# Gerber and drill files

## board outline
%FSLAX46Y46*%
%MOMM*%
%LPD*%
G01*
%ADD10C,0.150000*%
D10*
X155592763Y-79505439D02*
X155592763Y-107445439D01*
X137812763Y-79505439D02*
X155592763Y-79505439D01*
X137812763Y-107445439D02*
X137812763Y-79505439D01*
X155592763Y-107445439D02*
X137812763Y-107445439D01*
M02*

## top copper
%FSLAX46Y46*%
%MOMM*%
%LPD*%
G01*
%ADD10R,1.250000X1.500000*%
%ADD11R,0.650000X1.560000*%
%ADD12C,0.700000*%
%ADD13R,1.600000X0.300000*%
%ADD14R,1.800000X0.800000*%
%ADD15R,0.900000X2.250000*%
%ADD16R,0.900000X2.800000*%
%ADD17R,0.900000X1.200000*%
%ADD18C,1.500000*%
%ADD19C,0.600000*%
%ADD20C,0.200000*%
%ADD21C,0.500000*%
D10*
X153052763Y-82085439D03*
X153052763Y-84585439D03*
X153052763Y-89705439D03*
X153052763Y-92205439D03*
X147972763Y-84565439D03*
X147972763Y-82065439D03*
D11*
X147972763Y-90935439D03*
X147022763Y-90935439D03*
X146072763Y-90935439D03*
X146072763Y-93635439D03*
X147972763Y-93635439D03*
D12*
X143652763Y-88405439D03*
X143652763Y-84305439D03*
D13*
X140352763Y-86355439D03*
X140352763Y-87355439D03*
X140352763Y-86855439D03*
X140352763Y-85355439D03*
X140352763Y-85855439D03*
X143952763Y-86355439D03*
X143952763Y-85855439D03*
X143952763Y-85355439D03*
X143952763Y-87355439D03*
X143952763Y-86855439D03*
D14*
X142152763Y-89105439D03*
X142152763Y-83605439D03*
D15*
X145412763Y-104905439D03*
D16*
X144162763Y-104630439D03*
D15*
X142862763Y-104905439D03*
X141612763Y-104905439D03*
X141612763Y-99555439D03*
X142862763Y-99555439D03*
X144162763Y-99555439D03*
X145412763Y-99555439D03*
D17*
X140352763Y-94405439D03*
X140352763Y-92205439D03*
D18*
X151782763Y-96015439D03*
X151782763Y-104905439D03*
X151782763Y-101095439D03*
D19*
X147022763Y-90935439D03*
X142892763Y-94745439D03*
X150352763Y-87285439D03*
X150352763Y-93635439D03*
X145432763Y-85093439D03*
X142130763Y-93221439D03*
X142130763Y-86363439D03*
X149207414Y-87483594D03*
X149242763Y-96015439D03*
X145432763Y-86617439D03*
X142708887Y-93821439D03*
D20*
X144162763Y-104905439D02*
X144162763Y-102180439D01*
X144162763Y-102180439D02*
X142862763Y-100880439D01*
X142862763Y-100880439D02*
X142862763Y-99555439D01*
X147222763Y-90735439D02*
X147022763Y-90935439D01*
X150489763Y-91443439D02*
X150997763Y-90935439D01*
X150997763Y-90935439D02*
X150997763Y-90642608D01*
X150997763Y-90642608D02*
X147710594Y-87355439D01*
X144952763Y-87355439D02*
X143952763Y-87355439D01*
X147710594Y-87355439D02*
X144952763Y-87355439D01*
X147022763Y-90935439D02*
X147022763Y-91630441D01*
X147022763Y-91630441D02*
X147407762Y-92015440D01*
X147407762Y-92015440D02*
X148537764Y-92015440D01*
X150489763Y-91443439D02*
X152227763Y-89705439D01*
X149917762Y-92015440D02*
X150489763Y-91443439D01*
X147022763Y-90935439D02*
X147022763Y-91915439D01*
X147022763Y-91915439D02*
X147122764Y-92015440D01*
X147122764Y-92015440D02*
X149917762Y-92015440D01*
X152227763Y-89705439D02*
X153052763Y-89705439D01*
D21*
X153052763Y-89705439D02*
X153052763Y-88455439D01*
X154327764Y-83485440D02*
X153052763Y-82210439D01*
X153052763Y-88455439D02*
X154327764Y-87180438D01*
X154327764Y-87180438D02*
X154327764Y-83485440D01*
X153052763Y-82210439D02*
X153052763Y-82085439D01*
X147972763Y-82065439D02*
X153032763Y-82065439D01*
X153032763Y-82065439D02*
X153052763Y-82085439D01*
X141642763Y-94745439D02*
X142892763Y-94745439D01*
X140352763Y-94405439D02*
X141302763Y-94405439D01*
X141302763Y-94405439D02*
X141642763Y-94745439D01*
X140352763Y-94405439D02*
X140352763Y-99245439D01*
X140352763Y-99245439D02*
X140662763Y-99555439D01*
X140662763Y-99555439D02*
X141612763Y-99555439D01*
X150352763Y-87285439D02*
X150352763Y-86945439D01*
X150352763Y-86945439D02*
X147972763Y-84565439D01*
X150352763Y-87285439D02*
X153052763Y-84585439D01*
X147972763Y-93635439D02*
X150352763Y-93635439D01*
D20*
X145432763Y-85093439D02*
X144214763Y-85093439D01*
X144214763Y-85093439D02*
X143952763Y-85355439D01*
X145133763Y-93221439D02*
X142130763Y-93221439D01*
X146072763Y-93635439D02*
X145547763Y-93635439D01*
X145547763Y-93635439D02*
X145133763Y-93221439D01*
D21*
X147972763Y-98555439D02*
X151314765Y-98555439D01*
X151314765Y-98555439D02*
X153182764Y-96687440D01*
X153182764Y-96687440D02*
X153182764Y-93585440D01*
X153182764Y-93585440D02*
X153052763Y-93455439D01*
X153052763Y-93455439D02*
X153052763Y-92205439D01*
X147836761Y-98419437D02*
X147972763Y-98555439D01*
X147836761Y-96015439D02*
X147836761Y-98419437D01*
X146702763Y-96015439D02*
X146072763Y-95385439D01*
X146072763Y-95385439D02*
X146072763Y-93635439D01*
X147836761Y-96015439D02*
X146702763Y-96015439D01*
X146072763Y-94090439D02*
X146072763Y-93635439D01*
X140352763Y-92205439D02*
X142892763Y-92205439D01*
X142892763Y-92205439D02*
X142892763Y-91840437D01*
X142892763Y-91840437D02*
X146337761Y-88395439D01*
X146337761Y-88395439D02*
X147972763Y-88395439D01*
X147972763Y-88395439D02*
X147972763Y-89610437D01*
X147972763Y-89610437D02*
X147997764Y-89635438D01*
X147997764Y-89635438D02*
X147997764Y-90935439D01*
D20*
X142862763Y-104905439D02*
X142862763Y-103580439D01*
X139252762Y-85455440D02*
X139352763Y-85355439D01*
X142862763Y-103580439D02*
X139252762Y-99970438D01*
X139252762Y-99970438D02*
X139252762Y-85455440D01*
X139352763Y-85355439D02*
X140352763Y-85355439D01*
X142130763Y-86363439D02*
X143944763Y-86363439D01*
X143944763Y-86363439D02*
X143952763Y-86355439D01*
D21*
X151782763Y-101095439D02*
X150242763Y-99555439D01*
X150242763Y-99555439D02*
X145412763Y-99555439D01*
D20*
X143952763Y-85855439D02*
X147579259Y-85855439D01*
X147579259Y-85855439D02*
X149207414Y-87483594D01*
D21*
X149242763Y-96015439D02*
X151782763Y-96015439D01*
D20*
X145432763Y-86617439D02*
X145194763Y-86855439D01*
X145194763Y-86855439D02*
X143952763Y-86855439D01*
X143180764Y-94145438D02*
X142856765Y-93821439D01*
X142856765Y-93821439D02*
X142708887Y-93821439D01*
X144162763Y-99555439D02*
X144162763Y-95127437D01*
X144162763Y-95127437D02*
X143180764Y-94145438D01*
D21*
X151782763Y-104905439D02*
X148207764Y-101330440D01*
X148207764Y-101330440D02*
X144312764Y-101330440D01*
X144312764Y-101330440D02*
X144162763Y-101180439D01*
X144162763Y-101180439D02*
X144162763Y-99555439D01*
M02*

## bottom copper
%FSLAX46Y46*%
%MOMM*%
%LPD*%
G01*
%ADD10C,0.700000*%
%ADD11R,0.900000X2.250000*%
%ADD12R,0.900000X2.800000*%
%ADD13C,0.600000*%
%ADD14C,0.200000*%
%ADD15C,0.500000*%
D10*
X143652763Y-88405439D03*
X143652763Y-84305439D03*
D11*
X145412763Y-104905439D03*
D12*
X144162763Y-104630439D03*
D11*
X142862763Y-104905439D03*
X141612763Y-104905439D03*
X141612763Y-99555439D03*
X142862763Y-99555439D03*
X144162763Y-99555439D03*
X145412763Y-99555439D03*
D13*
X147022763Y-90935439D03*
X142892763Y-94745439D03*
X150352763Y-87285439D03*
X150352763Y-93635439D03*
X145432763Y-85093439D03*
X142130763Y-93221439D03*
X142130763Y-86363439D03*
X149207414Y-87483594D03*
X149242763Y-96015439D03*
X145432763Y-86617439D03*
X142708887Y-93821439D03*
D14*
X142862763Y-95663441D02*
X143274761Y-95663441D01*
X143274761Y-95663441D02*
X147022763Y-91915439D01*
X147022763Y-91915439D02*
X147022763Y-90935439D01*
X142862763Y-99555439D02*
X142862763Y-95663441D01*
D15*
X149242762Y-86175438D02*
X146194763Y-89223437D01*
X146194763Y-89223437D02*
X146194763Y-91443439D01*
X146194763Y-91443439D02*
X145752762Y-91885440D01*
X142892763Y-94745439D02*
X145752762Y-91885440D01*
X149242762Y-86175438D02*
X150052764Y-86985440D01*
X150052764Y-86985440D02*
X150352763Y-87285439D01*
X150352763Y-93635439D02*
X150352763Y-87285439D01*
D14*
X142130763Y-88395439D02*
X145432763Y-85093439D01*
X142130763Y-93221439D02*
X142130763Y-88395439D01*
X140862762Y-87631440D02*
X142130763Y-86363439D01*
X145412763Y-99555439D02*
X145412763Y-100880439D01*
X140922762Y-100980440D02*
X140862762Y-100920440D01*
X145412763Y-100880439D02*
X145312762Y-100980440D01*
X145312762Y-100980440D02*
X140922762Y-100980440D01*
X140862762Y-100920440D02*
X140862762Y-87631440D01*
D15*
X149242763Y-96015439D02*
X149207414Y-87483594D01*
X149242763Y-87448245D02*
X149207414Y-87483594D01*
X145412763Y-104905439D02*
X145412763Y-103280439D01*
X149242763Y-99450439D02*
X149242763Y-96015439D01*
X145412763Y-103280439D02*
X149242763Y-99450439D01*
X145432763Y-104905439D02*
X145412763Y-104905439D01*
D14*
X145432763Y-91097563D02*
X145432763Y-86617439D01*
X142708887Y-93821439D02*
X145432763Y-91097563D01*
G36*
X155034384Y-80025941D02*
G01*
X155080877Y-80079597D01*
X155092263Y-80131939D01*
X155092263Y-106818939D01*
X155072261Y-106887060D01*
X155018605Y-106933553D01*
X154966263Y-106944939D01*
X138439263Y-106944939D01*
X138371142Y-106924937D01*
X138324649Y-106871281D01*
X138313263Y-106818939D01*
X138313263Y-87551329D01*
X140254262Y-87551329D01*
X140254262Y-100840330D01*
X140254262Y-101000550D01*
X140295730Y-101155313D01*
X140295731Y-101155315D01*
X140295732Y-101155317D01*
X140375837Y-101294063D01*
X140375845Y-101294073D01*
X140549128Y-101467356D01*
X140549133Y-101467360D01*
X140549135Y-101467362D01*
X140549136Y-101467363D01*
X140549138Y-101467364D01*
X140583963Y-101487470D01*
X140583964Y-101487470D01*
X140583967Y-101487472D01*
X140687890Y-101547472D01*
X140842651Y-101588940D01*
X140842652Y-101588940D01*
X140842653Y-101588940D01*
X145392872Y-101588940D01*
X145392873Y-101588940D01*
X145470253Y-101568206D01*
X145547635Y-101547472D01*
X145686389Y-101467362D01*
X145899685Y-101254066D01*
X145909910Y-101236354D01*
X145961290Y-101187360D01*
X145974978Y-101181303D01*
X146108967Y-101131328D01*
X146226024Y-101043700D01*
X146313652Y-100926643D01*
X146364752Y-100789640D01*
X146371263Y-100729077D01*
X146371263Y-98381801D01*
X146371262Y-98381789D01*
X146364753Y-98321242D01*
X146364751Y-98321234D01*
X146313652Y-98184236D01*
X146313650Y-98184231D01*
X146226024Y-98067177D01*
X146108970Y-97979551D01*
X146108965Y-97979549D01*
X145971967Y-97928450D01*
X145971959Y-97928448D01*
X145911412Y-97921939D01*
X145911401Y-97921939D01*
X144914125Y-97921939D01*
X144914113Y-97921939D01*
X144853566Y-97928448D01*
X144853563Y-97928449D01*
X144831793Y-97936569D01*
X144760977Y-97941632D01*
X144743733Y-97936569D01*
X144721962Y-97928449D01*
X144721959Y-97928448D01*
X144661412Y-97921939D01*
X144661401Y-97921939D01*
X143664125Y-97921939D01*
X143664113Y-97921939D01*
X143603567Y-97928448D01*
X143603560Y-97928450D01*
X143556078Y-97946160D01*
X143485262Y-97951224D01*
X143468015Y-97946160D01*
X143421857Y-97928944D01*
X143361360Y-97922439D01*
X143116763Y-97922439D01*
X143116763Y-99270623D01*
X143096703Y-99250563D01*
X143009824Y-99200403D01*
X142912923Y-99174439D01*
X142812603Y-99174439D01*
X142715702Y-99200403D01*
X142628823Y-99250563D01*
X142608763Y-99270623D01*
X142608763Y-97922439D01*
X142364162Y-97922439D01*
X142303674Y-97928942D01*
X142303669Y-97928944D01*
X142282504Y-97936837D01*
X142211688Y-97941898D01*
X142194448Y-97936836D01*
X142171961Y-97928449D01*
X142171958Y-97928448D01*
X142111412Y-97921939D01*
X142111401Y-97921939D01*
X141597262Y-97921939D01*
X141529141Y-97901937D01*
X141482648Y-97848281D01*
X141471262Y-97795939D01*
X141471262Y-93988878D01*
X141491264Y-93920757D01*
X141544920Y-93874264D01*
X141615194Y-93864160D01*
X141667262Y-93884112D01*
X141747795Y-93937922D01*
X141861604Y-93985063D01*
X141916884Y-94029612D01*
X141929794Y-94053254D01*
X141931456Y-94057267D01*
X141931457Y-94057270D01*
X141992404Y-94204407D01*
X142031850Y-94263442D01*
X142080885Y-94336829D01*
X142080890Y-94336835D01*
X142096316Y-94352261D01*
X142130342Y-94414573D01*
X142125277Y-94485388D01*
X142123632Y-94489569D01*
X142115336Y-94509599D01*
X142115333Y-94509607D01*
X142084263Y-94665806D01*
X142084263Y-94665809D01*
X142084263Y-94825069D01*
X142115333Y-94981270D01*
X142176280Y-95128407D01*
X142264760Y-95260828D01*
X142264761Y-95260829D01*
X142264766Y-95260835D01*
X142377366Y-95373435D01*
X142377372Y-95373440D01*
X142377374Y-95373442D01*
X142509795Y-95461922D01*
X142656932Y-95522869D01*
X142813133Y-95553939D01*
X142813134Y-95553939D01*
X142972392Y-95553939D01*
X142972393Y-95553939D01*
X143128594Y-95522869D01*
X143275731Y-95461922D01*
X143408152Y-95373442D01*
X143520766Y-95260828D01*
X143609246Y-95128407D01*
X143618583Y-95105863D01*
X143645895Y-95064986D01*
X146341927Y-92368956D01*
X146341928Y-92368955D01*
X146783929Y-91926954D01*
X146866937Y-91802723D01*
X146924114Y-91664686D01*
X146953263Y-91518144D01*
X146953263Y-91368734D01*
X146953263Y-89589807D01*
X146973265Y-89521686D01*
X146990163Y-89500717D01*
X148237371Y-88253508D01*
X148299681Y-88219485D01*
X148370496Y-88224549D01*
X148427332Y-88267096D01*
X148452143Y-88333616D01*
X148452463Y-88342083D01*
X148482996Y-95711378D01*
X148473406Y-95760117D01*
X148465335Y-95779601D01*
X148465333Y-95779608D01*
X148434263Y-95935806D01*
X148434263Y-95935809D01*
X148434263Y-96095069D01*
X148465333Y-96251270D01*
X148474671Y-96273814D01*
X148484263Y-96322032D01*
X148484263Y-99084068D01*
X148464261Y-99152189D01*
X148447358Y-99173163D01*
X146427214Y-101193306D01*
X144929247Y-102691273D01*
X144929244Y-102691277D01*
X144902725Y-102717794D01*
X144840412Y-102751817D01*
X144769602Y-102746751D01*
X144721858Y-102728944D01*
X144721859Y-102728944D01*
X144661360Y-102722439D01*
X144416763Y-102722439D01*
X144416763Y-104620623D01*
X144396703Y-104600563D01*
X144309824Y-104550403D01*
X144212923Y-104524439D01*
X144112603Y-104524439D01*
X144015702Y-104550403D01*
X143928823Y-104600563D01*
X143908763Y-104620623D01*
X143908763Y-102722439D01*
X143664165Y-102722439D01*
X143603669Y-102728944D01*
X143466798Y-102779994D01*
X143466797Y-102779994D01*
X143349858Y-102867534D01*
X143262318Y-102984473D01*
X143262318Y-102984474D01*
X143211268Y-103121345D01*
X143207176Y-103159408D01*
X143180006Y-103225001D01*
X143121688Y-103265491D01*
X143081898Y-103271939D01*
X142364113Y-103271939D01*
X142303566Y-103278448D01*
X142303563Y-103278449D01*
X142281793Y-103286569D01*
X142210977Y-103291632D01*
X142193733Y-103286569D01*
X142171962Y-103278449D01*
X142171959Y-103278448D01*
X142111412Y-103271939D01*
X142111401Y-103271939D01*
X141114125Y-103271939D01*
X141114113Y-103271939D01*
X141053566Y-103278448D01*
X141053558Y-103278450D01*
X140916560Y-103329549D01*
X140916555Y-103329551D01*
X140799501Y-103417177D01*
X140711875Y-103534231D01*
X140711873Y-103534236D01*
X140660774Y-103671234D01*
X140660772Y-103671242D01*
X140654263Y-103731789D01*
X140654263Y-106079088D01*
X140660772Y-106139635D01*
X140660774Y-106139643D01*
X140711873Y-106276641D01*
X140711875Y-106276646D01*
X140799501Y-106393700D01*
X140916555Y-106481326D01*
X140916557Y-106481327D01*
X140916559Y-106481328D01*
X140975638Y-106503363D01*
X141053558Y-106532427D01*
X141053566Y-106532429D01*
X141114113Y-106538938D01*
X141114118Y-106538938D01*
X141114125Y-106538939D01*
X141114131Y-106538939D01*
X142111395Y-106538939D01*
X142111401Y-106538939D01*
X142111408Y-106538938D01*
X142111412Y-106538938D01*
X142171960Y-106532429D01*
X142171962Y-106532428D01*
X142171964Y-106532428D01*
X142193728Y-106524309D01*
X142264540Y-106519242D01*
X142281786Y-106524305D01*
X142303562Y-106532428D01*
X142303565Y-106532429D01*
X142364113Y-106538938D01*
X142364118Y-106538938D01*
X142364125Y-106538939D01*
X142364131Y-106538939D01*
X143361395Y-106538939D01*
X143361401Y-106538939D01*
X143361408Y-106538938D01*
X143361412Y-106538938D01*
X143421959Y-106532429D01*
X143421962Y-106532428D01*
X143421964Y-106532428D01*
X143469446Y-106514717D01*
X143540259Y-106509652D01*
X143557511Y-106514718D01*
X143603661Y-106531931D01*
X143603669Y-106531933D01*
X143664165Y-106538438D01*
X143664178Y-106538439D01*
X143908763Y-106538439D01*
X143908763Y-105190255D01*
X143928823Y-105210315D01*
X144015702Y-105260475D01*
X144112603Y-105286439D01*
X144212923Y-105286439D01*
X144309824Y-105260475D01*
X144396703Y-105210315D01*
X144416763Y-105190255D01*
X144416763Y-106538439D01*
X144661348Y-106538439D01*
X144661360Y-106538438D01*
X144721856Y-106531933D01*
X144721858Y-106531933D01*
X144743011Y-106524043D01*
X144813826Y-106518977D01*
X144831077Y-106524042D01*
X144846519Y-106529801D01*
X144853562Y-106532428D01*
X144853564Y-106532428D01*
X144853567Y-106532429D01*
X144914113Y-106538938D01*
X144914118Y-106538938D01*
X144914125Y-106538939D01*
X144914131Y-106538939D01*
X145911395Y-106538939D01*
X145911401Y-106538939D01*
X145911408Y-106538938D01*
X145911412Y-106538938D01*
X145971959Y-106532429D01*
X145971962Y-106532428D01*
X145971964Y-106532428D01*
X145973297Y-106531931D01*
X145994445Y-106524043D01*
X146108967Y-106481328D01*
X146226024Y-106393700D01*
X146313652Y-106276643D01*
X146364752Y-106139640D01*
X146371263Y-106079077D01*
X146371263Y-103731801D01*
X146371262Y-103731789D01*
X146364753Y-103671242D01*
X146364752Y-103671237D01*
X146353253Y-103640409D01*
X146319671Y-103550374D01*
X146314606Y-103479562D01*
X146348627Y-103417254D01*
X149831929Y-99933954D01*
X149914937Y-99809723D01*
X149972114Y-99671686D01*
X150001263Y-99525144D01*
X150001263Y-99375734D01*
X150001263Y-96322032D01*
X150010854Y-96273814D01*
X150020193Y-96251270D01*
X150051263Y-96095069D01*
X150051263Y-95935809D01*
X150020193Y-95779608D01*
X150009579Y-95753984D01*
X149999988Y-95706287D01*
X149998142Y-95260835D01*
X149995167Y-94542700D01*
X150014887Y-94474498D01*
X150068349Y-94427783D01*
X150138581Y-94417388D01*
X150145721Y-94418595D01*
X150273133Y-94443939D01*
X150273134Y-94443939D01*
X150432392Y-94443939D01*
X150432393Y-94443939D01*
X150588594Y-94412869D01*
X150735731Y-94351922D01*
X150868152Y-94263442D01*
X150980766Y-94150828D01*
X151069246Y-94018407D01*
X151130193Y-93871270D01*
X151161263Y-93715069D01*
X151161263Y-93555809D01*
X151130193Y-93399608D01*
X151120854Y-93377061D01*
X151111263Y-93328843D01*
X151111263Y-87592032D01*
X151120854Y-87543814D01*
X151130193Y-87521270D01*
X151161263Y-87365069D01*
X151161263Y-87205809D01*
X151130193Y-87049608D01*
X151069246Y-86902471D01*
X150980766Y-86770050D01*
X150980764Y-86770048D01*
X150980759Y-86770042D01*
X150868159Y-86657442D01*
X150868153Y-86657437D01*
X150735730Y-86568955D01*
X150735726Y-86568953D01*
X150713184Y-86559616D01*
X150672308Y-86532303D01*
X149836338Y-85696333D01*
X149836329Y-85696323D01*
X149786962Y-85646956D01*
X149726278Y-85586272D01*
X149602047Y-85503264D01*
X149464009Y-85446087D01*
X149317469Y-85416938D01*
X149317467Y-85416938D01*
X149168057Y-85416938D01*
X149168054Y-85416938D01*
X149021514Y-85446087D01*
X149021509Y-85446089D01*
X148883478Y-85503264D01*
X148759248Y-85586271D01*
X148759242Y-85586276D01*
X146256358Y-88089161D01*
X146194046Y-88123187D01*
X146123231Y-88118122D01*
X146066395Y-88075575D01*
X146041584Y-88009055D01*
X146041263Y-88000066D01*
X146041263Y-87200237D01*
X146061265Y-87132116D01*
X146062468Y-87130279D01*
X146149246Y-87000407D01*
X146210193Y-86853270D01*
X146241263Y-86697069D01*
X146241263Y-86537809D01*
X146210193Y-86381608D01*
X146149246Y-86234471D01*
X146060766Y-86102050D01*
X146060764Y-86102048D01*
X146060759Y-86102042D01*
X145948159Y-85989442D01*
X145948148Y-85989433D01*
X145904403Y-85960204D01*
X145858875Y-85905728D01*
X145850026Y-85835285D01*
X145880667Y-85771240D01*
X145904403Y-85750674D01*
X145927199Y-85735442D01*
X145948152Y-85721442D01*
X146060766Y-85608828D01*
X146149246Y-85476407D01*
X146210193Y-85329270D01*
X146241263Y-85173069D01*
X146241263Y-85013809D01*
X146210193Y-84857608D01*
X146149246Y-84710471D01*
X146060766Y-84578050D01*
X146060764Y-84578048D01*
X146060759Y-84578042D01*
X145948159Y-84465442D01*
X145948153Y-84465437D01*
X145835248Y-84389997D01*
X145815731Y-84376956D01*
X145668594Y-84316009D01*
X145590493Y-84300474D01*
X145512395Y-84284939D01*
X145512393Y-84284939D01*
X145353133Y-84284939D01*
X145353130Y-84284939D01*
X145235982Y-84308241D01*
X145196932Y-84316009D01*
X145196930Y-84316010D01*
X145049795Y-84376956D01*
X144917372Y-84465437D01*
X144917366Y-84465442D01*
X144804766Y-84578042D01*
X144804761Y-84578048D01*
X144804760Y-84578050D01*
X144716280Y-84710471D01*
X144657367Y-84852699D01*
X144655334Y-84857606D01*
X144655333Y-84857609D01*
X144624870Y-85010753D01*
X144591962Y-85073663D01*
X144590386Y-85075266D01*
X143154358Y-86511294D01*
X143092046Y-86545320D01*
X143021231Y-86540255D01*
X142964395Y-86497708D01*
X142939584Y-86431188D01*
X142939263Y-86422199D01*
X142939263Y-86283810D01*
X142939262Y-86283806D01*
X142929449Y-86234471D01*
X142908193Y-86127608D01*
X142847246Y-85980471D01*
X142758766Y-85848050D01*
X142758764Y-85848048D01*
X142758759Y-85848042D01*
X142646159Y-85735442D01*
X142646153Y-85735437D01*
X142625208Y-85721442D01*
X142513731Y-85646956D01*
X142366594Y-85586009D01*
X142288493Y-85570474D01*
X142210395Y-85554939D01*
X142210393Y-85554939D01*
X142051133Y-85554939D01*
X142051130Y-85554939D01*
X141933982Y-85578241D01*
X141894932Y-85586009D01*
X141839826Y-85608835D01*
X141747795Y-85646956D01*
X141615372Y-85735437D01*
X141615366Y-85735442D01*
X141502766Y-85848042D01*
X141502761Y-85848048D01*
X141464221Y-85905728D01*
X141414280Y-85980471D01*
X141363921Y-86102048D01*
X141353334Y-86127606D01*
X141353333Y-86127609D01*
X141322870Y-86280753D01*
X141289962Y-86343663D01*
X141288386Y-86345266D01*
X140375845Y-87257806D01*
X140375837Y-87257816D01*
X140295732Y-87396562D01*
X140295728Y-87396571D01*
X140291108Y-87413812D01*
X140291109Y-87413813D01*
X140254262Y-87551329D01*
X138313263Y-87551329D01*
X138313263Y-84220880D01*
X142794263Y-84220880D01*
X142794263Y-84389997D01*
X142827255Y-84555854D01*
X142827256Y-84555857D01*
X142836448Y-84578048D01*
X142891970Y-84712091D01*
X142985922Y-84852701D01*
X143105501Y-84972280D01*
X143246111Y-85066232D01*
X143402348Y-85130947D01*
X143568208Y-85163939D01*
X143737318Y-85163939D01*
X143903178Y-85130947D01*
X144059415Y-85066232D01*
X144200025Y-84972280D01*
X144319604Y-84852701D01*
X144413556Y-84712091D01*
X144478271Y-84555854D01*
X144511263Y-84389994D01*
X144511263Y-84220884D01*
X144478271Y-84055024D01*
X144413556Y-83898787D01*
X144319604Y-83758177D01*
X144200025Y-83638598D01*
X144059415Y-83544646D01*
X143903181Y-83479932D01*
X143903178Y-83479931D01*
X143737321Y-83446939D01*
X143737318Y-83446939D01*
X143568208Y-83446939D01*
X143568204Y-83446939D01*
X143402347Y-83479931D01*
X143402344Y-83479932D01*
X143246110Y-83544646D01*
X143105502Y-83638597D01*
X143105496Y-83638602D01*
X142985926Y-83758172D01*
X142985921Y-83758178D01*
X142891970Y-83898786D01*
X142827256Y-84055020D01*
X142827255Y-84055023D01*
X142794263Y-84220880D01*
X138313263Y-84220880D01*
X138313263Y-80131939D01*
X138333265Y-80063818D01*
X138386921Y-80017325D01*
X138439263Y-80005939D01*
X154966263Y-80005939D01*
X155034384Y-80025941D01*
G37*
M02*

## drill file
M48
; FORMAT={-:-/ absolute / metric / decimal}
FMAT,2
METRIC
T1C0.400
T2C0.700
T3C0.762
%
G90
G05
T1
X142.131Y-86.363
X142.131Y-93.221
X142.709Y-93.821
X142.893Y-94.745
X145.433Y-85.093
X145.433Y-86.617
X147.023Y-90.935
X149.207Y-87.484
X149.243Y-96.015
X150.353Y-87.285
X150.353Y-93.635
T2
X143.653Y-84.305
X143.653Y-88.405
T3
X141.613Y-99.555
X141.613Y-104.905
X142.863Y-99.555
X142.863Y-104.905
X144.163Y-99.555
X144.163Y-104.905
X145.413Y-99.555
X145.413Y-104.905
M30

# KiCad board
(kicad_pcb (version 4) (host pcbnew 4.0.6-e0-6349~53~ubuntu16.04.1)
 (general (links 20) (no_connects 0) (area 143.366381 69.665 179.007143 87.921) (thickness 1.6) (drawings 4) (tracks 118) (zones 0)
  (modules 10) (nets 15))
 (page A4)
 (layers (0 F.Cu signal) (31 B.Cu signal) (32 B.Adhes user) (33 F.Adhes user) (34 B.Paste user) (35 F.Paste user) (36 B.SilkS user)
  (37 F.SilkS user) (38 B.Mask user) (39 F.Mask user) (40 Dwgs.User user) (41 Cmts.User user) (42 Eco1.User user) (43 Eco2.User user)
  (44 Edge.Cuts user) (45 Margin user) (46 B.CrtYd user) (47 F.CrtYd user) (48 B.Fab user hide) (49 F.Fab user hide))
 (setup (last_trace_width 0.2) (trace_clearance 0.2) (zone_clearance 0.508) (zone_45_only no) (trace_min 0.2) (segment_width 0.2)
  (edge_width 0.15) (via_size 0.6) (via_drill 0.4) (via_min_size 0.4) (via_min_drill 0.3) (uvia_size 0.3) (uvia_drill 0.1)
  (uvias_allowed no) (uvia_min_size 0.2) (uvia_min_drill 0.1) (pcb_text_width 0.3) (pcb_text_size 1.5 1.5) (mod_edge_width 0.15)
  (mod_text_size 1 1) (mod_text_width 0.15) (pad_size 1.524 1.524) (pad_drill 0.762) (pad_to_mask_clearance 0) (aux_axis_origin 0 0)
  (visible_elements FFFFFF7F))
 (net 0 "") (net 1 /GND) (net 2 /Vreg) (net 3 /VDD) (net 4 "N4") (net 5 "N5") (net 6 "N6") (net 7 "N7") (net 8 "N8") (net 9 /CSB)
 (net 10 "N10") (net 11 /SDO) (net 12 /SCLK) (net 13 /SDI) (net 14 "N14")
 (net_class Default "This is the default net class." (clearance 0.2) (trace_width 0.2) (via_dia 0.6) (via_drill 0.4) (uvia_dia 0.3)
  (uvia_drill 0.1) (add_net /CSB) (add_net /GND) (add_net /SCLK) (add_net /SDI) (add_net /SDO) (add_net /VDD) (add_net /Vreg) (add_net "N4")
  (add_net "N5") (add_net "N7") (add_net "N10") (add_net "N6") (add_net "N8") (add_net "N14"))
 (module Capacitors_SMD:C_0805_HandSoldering (layer F.Cu) (at 153.052763 83.335439 270)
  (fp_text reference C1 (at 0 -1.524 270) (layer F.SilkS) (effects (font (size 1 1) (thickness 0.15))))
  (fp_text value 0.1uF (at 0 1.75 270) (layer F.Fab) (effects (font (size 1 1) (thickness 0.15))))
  (pad 1 smd rect (at -1.25 0 270) (size 1.5 1.25) (layers F.Cu F.Paste F.Mask) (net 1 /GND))
  (pad 2 smd rect (at 1.25 0 270) (size 1.5 1.25) (layers F.Cu F.Paste F.Mask) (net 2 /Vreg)))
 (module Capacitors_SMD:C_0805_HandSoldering (layer F.Cu) (at 153.052763 90.955439 270)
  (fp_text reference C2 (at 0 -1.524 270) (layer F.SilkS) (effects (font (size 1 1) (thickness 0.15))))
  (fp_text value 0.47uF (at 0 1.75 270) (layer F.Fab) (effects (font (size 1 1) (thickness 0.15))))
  (pad 1 smd rect (at -1.25 0 270) (size 1.5 1.25) (layers F.Cu F.Paste F.Mask) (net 1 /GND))
  (pad 2 smd rect (at 1.25 0 270) (size 1.5 1.25) (layers F.Cu F.Paste F.Mask) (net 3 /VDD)))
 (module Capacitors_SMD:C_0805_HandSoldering (layer F.Cu) (at 147.972763 83.315439 90)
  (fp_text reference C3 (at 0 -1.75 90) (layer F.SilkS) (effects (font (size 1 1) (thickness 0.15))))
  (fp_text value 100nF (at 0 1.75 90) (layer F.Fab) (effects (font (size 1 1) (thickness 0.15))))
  (pad 1 smd rect (at -1.25 0 90) (size 1.5 1.25) (layers F.Cu F.Paste F.Mask) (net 2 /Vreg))
  (pad 2 smd rect (at 1.25 0 90) (size 1.5 1.25) (layers F.Cu F.Paste F.Mask) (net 1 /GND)))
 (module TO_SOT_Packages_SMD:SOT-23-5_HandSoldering (layer F.Cu) (at 147.022763 92.285439 270)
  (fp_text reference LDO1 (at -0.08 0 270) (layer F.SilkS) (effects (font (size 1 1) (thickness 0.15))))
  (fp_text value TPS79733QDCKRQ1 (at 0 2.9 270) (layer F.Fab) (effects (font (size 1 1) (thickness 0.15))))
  (pad 1 smd rect (at -1.35 -0.95 270) (size 1.56 0.65) (layers F.Cu F.Paste F.Mask) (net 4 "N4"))
  (pad 2 smd rect (at -1.35 0 270) (size 1.56 0.65) (layers F.Cu F.Paste F.Mask) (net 1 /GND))
  (pad 3 smd rect (at -1.35 0.95 270) (size 1.56 0.65) (layers F.Cu F.Paste F.Mask) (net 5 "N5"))
  (pad 4 smd rect (at 1.35 0.95 270) (size 1.56 0.65) (layers F.Cu F.Paste F.Mask) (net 3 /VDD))
  (pad 5 smd rect (at 1.35 -0.95 270) (size 1.56 0.65) (layers F.Cu F.Paste F.Mask) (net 2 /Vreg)))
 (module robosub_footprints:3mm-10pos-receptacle (layer F.Cu) (at 142.152763 86.355439 270)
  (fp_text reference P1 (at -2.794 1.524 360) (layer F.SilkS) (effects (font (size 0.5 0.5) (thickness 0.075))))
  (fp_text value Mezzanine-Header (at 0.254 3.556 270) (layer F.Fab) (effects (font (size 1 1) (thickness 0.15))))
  (pad "" thru_hole circle (at 2.05 -1.5 270) (size 0.7 0.7) (drill 0.7) (layers *.Cu *.Mask))
  (pad "" thru_hole circle (at -2.05 -1.5 270) (size 0.7 0.7) (drill 0.7) (layers *.Cu *.Mask))
  (pad 6 smd rect (at 0 1.8 270) (size 0.3 1.6) (layers F.Cu F.Paste F.Mask) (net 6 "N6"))
  (pad 10 smd rect (at 1 1.8 270) (size 0.3 1.6) (layers F.Cu F.Paste F.Mask) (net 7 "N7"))
  (pad 8 smd rect (at 0.5 1.8 270) (size 0.3 1.6) (layers F.Cu F.Paste F.Mask) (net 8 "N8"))
  (pad 2 smd rect (at -1 1.8 270) (size 0.3 1.6) (layers F.Cu F.Paste F.Mask) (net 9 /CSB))
  (pad 4 smd rect (at -0.5 1.8 270) (size 0.3 1.6) (layers F.Cu F.Paste F.Mask) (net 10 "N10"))
  (pad 5 smd rect (at 0 -1.8 270) (size 0.3 1.6) (layers F.Cu F.Paste F.Mask) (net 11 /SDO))
  (pad 3 smd rect (at -0.5 -1.8 270) (size 0.3 1.6) (layers F.Cu F.Paste F.Mask) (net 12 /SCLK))
  (pad 1 smd rect (at -1 -1.8 270) (size 0.3 1.6) (layers F.Cu F.Paste F.Mask) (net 3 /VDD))
  (pad 9 smd rect (at 1 -1.8 270) (size 0.3 1.6) (layers F.Cu F.Paste F.Mask) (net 1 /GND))
  (pad 7 smd rect (at 0.5 -1.8 270) (size 0.3 1.6) (layers F.Cu F.Paste F.Mask) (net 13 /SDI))
  (pad "" smd rect (at 2.75 0 270) (size 0.8 1.8) (layers F.Cu F.Paste F.Mask))
  (pad "" smd rect (at -2.75 0 270) (size 0.8 1.8) (layers F.Cu F.Paste F.Mask)))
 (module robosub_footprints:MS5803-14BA (layer F.Cu) (at 141.612763 99.555439 270)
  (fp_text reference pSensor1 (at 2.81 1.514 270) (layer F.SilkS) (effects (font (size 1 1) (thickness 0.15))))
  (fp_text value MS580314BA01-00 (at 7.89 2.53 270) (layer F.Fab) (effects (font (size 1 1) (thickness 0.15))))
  (pad 1 thru_hole rect (at 5.35 -3.8 270) (size 2.25 0.9) (drill 0.762) (layers *.Cu *.Mask) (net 12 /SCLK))
  (pad 2 thru_hole rect (at 5.35 -2.55 270) (size 2.8 0.9) (drill 0.762 (offset -0.275 0)) (layers *.Cu *.Mask) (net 1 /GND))
  (pad 3 thru_hole rect (at 5.35 -1.25 270) (size 2.25 0.9) (drill 0.762) (layers *.Cu *.Mask) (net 9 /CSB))
  (pad 4 thru_hole rect (at 5.35 0 270) (size 2.25 0.9) (drill 0.762) (layers *.Cu *.Mask) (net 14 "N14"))
  (pad 5 thru_hole rect (at 0 0 270) (size 2.25 0.9) (drill 0.762) (layers *.Cu *.Mask) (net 2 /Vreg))
  (pad 6 thru_hole rect (at 0 -1.25 270) (size 2.25 0.9) (drill 0.762) (layers *.Cu *.Mask) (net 1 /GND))
  (pad 7 thru_hole rect (at 0 -2.55 270) (size 2.25 0.9) (drill 0.762) (layers *.Cu *.Mask) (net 13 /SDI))
  (pad 8 thru_hole rect (at 0 -3.8 270) (size 2.25 0.9) (drill 0.762) (layers *.Cu *.Mask) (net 11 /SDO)))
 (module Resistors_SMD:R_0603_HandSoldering (layer F.Cu) (at 140.352763 93.305439 90)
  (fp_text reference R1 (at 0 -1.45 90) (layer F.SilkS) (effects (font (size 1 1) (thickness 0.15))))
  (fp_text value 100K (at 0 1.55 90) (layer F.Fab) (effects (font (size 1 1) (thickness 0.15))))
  (pad 1 smd rect (at -1.1 0 90) (size 1.2 0.9) (layers F.Cu F.Paste F.Mask) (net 2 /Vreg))
  (pad 2 smd rect (at 1.1 0 90) (size 1.2 0.9) (layers F.Cu F.Paste F.Mask) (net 4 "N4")))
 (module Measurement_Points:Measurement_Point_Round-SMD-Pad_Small (layer F.Cu) (at 151.782763 96.015439 270)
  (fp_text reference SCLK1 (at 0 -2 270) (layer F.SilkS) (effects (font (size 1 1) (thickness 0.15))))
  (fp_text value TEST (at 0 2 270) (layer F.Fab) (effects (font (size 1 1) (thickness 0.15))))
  (pad 1 smd circle (at 0 0 270) (size 1.5 1.5) (layers F.Cu F.Mask) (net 12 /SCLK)))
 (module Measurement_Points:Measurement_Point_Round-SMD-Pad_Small (layer F.Cu) (at 151.782763 104.905439 270)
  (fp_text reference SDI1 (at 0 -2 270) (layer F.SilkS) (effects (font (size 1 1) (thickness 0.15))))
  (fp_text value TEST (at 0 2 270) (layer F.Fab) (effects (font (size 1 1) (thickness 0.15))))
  (pad 1 smd circle (at 0 0 270) (size 1.5 1.5) (layers F.Cu F.Mask) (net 13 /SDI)))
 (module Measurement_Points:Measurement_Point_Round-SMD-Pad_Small (layer F.Cu) (at 151.782763 101.095439 270)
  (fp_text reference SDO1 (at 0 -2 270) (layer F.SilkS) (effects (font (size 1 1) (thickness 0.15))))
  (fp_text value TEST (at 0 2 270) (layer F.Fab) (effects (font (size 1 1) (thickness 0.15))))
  (pad 1 smd circle (at 0 0 270) (size 1.5 1.5) (layers F.Cu F.Mask) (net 11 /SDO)))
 (gr_line (start 155.592763 79.505439) (end 155.592763 107.445439) (angle 90) (layer Edge.Cuts) (width 0.15))
 (gr_line (start 137.812763 79.505439) (end 155.592763 79.505439) (angle 90) (layer Edge.Cuts) (width 0.15))
 (gr_line (start 137.812763 107.445439) (end 137.812763 79.505439) (angle 90) (layer Edge.Cuts) (width 0.15))
 (gr_line (start 155.592763 107.445439) (end 137.812763 107.445439) (angle 90) (layer Edge.Cuts) (width 0.15))
 (segment (start 142.862763 95.663441) (end 143.274761 95.663441) (width 0.2) (layer B.Cu) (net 1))
 (segment (start 143.274761 95.663441) (end 147.022763 91.915439) (width 0.2) (layer B.Cu) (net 1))
 (segment (start 147.022763 91.915439) (end 147.022763 90.935439) (width 0.2) (layer B.Cu) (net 1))
 (via (at 147.022763 90.935439) (size 0.6) (drill 0.4) (layers F.Cu B.Cu) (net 1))
 (segment (start 144.162763 104.905439) (end 144.162763 102.180439) (width 0.2) (layer F.Cu) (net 1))
 (segment (start 144.162763 102.180439) (end 142.862763 100.880439) (width 0.2) (layer F.Cu) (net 1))
 (segment (start 142.862763 100.880439) (end 142.862763 99.555439) (width 0.2) (layer F.Cu) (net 1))
 (segment (start 147.222763 90.735439) (end 147.022763 90.935439) (width 0.2) (layer F.Cu) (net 1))
 (segment (start 142.862763 99.555439) (end 142.862763 95.663441) (width 0.2) (layer B.Cu) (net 1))
 (segment (start 150.489763 91.443439) (end 150.997763 90.935439) (width 0.2) (layer F.Cu) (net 1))
 (segment (start 150.997763 90.935439) (end 150.997763 90.642608) (width 0.2) (layer F.Cu) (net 1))
 (segment (start 150.997763 90.642608) (end 147.710594 87.355439) (width 0.2) (layer F.Cu) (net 1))
 (segment (start 144.952763 87.355439) (end 143.952763 87.355439) (width 0.2) (layer F.Cu) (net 1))
 (segment (start 147.710594 87.355439) (end 144.952763 87.355439) (width 0.2) (layer F.Cu) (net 1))
 (segment (start 147.022763 90.935439) (end 147.022763 91.630441) (width 0.2) (layer F.Cu) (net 1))
 (segment (start 147.022763 91.630441) (end 147.407762 92.01544) (width 0.2) (layer F.Cu) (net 1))
 (segment (start 147.407762 92.01544) (end 148.537764 92.01544) (width 0.2) (layer F.Cu) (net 1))
 (segment (start 150.489763 91.443439) (end 152.227763 89.705439) (width 0.2) (layer F.Cu) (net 1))
 (segment (start 149.917762 92.01544) (end 150.489763 91.443439) (width 0.2) (layer F.Cu) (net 1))
 (segment (start 147.022763 90.935439) (end 147.022763 91.915439) (width 0.2) (layer F.Cu) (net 1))
 (segment (start 147.022763 91.915439) (end 147.122764 92.01544) (width 0.2) (layer F.Cu) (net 1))
 (segment (start 147.122764 92.01544) (end 149.917762 92.01544) (width 0.2) (layer F.Cu) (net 1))
 (segment (start 152.227763 89.705439) (end 153.052763 89.705439) (width 0.2) (layer F.Cu) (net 1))
 (segment (start 153.052763 89.705439) (end 153.052763 88.455439) (width 0.5) (layer F.Cu) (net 1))
 (segment (start 154.327764 83.48544) (end 153.052763 82.210439) (width 0.5) (layer F.Cu) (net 1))
 (segment (start 153.052763 88.455439) (end 154.327764 87.180438) (width 0.5) (layer F.Cu) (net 1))
 (segment (start 154.327764 87.180438) (end 154.327764 83.48544) (width 0.5) (layer F.Cu) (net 1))
 (segment (start 153.052763 82.210439) (end 153.052763 82.085439) (width 0.5) (layer F.Cu) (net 1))
 (segment (start 147.972763 82.065439) (end 153.032763 82.065439) (width 0.5) (layer F.Cu) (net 1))
 (segment (start 153.032763 82.065439) (end 153.052763 82.085439) (width 0.5) (layer F.Cu) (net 1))
 (segment (start 149.242762 86.175438) (end 146.194763 89.223437) (width 0.5) (layer B.Cu) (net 2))
 (segment (start 146.194763 89.223437) (end 146.194763 91.443439) (width 0.5) (layer B.Cu) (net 2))
 (segment (start 146.194763 91.443439) (end 145.752762 91.88544) (width 0.5) (layer B.Cu) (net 2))
 (segment (start 142.892763 94.745439) (end 145.752762 91.88544) (width 0.5) (layer B.Cu) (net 2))
 (segment (start 149.242762 86.175438) (end 150.052764 86.98544) (width 0.5) (layer B.Cu) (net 2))
 (segment (start 150.052764 86.98544) (end 150.352763 87.285439) (width 0.5) (layer B.Cu) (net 2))
 (via (at 142.892763 94.745439) (size 0.6) (drill 0.4) (layers F.Cu B.Cu) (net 2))
 (segment (start 141.642763 94.745439) (end 142.892763 94.745439) (width 0.5) (layer F.Cu) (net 2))
 (segment (start 140.352763 94.405439) (end 141.302763 94.405439) (width 0.5) (layer F.Cu) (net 2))
 (segment (start 141.302763 94.405439) (end 141.642763 94.745439) (width 0.5) (layer F.Cu) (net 2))
 (segment (start 140.352763 94.405439) (end 140.352763 99.245439) (width 0.5) (layer F.Cu) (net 2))
 (segment (start 140.352763 99.245439) (end 140.662763 99.555439) (width 0.5) (layer F.Cu) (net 2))
 (segment (start 140.662763 99.555439) (end 141.612763 99.555439) (width 0.5) (layer F.Cu) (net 2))
 (segment (start 150.352763 87.285439) (end 150.352763 86.945439) (width 0.5) (layer F.Cu) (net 2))
 (segment (start 150.352763 86.945439) (end 147.972763 84.565439) (width 0.5) (layer F.Cu) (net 2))
 (segment (start 150.352763 87.285439) (end 153.052763 84.585439) (width 0.5) (layer F.Cu) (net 2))
 (via (at 150.352763 87.285439) (size 0.6) (drill 0.4) (layers F.Cu B.Cu) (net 2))
 (segment (start 150.352763 93.635439) (end 150.352763 87.285439) (width 0.5) (layer B.Cu) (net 2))
 (via (at 150.352763 93.635439) (size 0.6) (drill 0.4) (layers F.Cu B.Cu) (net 2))
 (segment (start 147.972763 93.635439) (end 150.352763 93.635439) (width 0.5) (layer F.Cu) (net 2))
 (segment (start 145.432763 85.093439) (end 144.214763 85.093439) (width 0.2) (layer F.Cu) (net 3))
 (segment (start 144.214763 85.093439) (end 143.952763 85.355439) (width 0.2) (layer F.Cu) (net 3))
 (segment (start 142.130763 88.395439) (end 145.432763 85.093439) (width 0.2) (layer B.Cu) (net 3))
 (via (at 145.432763 85.093439) (size 0.6) (drill 0.4) (layers F.Cu B.Cu) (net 3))
 (segment (start 142.130763 93.221439) (end 142.130763 88.395439) (width 0.2) (layer B.Cu) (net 3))
 (segment (start 145.133763 93.221439) (end 142.130763 93.221439) (width 0.2) (layer F.Cu) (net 3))
 (via (at 142.130763 93.221439) (size 0.6) (drill 0.4) (layers F.Cu B.Cu) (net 3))
 (segment (start 146.072763 93.635439) (end 145.547763 93.635439) (width 0.2) (layer F.Cu) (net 3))
 (segment (start 145.547763 93.635439) (end 145.133763 93.221439) (width 0.2) (layer F.Cu) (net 3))
 (segment (start 147.972763 98.555439) (end 151.314765 98.555439) (width 0.5) (layer F.Cu) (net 3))
 (segment (start 151.314765 98.555439) (end 153.182764 96.68744) (width 0.5) (layer F.Cu) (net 3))
 (segment (start 153.182764 96.68744) (end 153.182764 93.58544) (width 0.5) (layer F.Cu) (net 3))
 (segment (start 153.182764 93.58544) (end 153.052763 93.455439) (width 0.5) (layer F.Cu) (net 3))
 (segment (start 153.052763 93.455439) (end 153.052763 92.205439) (width 0.5) (layer F.Cu) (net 3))
 (segment (start 147.836761 98.419437) (end 147.972763 98.555439) (width 0.5) (layer F.Cu) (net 3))
 (segment (start 147.836761 96.015439) (end 147.836761 98.419437) (width 0.5) (layer F.Cu) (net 3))
 (segment (start 146.702763 96.015439) (end 146.072763 95.385439) (width 0.5) (layer F.Cu) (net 3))
 (segment (start 146.072763 95.385439) (end 146.072763 93.635439) (width 0.5) (layer F.Cu) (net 3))
 (segment (start 147.836761 96.015439) (end 146.702763 96.015439) (width 0.5) (layer F.Cu) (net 3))
 (segment (start 146.072763 94.090439) (end 146.072763 93.635439) (width 0.5) (layer F.Cu) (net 3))
 (segment (start 140.352763 92.205439) (end 142.892763 92.205439) (width 0.5) (layer F.Cu) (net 4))
 (segment (start 142.892763 92.205439) (end 142.892763 91.840437) (width 0.5) (layer F.Cu) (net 4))
 (segment (start 142.892763 91.840437) (end 146.337761 88.395439) (width 0.5) (layer F.Cu) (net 4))
 (segment (start 146.337761 88.395439) (end 147.972763 88.395439) (width 0.5) (layer F.Cu) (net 4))
 (segment (start 147.972763 88.395439) (end 147.972763 89.610437) (width 0.5) (layer F.Cu) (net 4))
 (segment (start 147.972763 89.610437) (end 147.997764 89.635438) (width 0.5) (layer F.Cu) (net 4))
 (segment (start 147.997764 89.635438) (end 147.997764 90.935439) (width 0.5) (layer F.Cu) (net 4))
 (segment (start 142.862763 104.905439) (end 142.862763 103.580439) (width 0.2) (layer F.Cu) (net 9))
 (segment (start 139.252762 85.45544) (end 139.352763 85.355439) (width 0.2) (layer F.Cu) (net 9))
 (segment (start 142.862763 103.580439) (end 139.252762 99.970438) (width 0.2) (layer F.Cu) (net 9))
 (segment (start 139.252762 99.970438) (end 139.252762 85.45544) (width 0.2) (layer F.Cu) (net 9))
 (segment (start 139.352763 85.355439) (end 140.352763 85.355439) (width 0.2) (layer F.Cu) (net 9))
 (segment (start 142.130763 86.363439) (end 143.944763 86.363439) (width 0.2) (layer F.Cu) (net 11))
 (segment (start 143.944763 86.363439) (end 143.952763 86.355439) (width 0.2) (layer F.Cu) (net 11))
 (segment (start 140.862762 87.63144) (end 142.130763 86.363439) (width 0.2) (layer B.Cu) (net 11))
 (via (at 142.130763 86.363439) (size 0.6) (drill 0.4) (layers F.Cu B.Cu) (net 11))
 (segment (start 145.412763 99.555439) (end 145.412763 100.880439) (width 0.2) (layer B.Cu) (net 11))
 (segment (start 140.922762 100.98044) (end 140.862762 100.92044) (width 0.2) (layer B.Cu) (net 11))
 (segment (start 145.412763 100.880439) (end 145.312762 100.98044) (width 0.2) (layer B.Cu) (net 11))
 (segment (start 145.312762 100.98044) (end 140.922762 100.98044) (width 0.2) (layer B.Cu) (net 11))
 (segment (start 140.862762 100.92044) (end 140.862762 87.63144) (width 0.2) (layer B.Cu) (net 11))
 (segment (start 151.782763 101.095439) (end 150.242763 99.555439) (width 0.5) (layer F.Cu) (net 11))
 (segment (start 150.242763 99.555439) (end 145.412763 99.555439) (width 0.5) (layer F.Cu) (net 11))
 (segment (start 143.952763 85.855439) (end 147.579259 85.855439) (width 0.2) (layer F.Cu) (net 12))
 (segment (start 147.579259 85.855439) (end 149.207414 87.483594) (width 0.2) (layer F.Cu) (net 12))
 (segment (start 149.242763 96.015439) (end 149.207414 87.483594) (width 0.5) (layer B.Cu) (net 12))
 (segment (start 149.242763 87.448245) (end 149.207414 87.483594) (width 0.5) (layer B.Cu) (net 12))
 (via (at 149.207414 87.483594) (size 0.6) (drill 0.4) (layers F.Cu B.Cu) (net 12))
 (segment (start 149.242763 96.015439) (end 151.782763 96.015439) (width 0.5) (layer F.Cu) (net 12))
 (segment (start 145.412763 104.905439) (end 145.412763 103.280439) (width 0.5) (layer B.Cu) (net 12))
 (segment (start 149.242763 99.450439) (end 149.242763 96.015439) (width 0.5) (layer B.Cu) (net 12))
 (segment (start 145.412763 103.280439) (end 149.242763 99.450439) (width 0.5) (layer B.Cu) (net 12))
 (via (at 149.242763 96.015439) (size 0.6) (drill 0.4) (layers F.Cu B.Cu) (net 12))
 (segment (start 145.432763 104.905439) (end 145.412763 104.905439) (width 0.5) (layer B.Cu) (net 12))
 (segment (start 145.432763 86.617439) (end 145.194763 86.855439) (width 0.2) (layer F.Cu) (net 13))
 (segment (start 145.194763 86.855439) (end 143.952763 86.855439) (width 0.2) (layer F.Cu) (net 13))
 (segment (start 145.432763 91.097563) (end 145.432763 86.617439) (width 0.2) (layer B.Cu) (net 13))
 (via (at 145.432763 86.617439) (size 0.6) (drill 0.4) (layers F.Cu B.Cu) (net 13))
 (segment (start 142.708887 93.821439) (end 145.432763 91.097563) (width 0.2) (layer B.Cu) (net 13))
 (segment (start 143.180764 94.145438) (end 142.856765 93.821439) (width 0.2) (layer F.Cu) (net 13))
 (segment (start 142.856765 93.821439) (end 142.708887 93.821439) (width 0.2) (layer F.Cu) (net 13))
 (via (at 142.708887 93.821439) (size 0.6) (drill 0.4) (layers F.Cu B.Cu) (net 13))
 (segment (start 144.162763 99.555439) (end 144.162763 95.127437) (width 0.2) (layer F.Cu) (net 13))
 (segment (start 144.162763 95.127437) (end 143.180764 94.145438) (width 0.2) (layer F.Cu) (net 13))
 (segment (start 151.782763 104.905439) (end 148.207764 101.33044) (width 0.5) (layer F.Cu) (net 13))
 (segment (start 148.207764 101.33044) (end 144.312764 101.33044) (width 0.5) (layer F.Cu) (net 13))
 (segment (start 144.312764 101.33044) (end 144.162763 101.180439) (width 0.5) (layer F.Cu) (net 13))
 (segment (start 144.162763 101.180439) (end 144.162763 99.555439) (width 0.5) (layer F.Cu) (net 13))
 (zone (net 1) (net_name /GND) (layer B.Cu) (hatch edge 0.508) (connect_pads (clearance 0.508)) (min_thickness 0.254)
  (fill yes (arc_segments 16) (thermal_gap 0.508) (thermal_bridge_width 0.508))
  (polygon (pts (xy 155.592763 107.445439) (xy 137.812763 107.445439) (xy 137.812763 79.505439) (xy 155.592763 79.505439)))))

